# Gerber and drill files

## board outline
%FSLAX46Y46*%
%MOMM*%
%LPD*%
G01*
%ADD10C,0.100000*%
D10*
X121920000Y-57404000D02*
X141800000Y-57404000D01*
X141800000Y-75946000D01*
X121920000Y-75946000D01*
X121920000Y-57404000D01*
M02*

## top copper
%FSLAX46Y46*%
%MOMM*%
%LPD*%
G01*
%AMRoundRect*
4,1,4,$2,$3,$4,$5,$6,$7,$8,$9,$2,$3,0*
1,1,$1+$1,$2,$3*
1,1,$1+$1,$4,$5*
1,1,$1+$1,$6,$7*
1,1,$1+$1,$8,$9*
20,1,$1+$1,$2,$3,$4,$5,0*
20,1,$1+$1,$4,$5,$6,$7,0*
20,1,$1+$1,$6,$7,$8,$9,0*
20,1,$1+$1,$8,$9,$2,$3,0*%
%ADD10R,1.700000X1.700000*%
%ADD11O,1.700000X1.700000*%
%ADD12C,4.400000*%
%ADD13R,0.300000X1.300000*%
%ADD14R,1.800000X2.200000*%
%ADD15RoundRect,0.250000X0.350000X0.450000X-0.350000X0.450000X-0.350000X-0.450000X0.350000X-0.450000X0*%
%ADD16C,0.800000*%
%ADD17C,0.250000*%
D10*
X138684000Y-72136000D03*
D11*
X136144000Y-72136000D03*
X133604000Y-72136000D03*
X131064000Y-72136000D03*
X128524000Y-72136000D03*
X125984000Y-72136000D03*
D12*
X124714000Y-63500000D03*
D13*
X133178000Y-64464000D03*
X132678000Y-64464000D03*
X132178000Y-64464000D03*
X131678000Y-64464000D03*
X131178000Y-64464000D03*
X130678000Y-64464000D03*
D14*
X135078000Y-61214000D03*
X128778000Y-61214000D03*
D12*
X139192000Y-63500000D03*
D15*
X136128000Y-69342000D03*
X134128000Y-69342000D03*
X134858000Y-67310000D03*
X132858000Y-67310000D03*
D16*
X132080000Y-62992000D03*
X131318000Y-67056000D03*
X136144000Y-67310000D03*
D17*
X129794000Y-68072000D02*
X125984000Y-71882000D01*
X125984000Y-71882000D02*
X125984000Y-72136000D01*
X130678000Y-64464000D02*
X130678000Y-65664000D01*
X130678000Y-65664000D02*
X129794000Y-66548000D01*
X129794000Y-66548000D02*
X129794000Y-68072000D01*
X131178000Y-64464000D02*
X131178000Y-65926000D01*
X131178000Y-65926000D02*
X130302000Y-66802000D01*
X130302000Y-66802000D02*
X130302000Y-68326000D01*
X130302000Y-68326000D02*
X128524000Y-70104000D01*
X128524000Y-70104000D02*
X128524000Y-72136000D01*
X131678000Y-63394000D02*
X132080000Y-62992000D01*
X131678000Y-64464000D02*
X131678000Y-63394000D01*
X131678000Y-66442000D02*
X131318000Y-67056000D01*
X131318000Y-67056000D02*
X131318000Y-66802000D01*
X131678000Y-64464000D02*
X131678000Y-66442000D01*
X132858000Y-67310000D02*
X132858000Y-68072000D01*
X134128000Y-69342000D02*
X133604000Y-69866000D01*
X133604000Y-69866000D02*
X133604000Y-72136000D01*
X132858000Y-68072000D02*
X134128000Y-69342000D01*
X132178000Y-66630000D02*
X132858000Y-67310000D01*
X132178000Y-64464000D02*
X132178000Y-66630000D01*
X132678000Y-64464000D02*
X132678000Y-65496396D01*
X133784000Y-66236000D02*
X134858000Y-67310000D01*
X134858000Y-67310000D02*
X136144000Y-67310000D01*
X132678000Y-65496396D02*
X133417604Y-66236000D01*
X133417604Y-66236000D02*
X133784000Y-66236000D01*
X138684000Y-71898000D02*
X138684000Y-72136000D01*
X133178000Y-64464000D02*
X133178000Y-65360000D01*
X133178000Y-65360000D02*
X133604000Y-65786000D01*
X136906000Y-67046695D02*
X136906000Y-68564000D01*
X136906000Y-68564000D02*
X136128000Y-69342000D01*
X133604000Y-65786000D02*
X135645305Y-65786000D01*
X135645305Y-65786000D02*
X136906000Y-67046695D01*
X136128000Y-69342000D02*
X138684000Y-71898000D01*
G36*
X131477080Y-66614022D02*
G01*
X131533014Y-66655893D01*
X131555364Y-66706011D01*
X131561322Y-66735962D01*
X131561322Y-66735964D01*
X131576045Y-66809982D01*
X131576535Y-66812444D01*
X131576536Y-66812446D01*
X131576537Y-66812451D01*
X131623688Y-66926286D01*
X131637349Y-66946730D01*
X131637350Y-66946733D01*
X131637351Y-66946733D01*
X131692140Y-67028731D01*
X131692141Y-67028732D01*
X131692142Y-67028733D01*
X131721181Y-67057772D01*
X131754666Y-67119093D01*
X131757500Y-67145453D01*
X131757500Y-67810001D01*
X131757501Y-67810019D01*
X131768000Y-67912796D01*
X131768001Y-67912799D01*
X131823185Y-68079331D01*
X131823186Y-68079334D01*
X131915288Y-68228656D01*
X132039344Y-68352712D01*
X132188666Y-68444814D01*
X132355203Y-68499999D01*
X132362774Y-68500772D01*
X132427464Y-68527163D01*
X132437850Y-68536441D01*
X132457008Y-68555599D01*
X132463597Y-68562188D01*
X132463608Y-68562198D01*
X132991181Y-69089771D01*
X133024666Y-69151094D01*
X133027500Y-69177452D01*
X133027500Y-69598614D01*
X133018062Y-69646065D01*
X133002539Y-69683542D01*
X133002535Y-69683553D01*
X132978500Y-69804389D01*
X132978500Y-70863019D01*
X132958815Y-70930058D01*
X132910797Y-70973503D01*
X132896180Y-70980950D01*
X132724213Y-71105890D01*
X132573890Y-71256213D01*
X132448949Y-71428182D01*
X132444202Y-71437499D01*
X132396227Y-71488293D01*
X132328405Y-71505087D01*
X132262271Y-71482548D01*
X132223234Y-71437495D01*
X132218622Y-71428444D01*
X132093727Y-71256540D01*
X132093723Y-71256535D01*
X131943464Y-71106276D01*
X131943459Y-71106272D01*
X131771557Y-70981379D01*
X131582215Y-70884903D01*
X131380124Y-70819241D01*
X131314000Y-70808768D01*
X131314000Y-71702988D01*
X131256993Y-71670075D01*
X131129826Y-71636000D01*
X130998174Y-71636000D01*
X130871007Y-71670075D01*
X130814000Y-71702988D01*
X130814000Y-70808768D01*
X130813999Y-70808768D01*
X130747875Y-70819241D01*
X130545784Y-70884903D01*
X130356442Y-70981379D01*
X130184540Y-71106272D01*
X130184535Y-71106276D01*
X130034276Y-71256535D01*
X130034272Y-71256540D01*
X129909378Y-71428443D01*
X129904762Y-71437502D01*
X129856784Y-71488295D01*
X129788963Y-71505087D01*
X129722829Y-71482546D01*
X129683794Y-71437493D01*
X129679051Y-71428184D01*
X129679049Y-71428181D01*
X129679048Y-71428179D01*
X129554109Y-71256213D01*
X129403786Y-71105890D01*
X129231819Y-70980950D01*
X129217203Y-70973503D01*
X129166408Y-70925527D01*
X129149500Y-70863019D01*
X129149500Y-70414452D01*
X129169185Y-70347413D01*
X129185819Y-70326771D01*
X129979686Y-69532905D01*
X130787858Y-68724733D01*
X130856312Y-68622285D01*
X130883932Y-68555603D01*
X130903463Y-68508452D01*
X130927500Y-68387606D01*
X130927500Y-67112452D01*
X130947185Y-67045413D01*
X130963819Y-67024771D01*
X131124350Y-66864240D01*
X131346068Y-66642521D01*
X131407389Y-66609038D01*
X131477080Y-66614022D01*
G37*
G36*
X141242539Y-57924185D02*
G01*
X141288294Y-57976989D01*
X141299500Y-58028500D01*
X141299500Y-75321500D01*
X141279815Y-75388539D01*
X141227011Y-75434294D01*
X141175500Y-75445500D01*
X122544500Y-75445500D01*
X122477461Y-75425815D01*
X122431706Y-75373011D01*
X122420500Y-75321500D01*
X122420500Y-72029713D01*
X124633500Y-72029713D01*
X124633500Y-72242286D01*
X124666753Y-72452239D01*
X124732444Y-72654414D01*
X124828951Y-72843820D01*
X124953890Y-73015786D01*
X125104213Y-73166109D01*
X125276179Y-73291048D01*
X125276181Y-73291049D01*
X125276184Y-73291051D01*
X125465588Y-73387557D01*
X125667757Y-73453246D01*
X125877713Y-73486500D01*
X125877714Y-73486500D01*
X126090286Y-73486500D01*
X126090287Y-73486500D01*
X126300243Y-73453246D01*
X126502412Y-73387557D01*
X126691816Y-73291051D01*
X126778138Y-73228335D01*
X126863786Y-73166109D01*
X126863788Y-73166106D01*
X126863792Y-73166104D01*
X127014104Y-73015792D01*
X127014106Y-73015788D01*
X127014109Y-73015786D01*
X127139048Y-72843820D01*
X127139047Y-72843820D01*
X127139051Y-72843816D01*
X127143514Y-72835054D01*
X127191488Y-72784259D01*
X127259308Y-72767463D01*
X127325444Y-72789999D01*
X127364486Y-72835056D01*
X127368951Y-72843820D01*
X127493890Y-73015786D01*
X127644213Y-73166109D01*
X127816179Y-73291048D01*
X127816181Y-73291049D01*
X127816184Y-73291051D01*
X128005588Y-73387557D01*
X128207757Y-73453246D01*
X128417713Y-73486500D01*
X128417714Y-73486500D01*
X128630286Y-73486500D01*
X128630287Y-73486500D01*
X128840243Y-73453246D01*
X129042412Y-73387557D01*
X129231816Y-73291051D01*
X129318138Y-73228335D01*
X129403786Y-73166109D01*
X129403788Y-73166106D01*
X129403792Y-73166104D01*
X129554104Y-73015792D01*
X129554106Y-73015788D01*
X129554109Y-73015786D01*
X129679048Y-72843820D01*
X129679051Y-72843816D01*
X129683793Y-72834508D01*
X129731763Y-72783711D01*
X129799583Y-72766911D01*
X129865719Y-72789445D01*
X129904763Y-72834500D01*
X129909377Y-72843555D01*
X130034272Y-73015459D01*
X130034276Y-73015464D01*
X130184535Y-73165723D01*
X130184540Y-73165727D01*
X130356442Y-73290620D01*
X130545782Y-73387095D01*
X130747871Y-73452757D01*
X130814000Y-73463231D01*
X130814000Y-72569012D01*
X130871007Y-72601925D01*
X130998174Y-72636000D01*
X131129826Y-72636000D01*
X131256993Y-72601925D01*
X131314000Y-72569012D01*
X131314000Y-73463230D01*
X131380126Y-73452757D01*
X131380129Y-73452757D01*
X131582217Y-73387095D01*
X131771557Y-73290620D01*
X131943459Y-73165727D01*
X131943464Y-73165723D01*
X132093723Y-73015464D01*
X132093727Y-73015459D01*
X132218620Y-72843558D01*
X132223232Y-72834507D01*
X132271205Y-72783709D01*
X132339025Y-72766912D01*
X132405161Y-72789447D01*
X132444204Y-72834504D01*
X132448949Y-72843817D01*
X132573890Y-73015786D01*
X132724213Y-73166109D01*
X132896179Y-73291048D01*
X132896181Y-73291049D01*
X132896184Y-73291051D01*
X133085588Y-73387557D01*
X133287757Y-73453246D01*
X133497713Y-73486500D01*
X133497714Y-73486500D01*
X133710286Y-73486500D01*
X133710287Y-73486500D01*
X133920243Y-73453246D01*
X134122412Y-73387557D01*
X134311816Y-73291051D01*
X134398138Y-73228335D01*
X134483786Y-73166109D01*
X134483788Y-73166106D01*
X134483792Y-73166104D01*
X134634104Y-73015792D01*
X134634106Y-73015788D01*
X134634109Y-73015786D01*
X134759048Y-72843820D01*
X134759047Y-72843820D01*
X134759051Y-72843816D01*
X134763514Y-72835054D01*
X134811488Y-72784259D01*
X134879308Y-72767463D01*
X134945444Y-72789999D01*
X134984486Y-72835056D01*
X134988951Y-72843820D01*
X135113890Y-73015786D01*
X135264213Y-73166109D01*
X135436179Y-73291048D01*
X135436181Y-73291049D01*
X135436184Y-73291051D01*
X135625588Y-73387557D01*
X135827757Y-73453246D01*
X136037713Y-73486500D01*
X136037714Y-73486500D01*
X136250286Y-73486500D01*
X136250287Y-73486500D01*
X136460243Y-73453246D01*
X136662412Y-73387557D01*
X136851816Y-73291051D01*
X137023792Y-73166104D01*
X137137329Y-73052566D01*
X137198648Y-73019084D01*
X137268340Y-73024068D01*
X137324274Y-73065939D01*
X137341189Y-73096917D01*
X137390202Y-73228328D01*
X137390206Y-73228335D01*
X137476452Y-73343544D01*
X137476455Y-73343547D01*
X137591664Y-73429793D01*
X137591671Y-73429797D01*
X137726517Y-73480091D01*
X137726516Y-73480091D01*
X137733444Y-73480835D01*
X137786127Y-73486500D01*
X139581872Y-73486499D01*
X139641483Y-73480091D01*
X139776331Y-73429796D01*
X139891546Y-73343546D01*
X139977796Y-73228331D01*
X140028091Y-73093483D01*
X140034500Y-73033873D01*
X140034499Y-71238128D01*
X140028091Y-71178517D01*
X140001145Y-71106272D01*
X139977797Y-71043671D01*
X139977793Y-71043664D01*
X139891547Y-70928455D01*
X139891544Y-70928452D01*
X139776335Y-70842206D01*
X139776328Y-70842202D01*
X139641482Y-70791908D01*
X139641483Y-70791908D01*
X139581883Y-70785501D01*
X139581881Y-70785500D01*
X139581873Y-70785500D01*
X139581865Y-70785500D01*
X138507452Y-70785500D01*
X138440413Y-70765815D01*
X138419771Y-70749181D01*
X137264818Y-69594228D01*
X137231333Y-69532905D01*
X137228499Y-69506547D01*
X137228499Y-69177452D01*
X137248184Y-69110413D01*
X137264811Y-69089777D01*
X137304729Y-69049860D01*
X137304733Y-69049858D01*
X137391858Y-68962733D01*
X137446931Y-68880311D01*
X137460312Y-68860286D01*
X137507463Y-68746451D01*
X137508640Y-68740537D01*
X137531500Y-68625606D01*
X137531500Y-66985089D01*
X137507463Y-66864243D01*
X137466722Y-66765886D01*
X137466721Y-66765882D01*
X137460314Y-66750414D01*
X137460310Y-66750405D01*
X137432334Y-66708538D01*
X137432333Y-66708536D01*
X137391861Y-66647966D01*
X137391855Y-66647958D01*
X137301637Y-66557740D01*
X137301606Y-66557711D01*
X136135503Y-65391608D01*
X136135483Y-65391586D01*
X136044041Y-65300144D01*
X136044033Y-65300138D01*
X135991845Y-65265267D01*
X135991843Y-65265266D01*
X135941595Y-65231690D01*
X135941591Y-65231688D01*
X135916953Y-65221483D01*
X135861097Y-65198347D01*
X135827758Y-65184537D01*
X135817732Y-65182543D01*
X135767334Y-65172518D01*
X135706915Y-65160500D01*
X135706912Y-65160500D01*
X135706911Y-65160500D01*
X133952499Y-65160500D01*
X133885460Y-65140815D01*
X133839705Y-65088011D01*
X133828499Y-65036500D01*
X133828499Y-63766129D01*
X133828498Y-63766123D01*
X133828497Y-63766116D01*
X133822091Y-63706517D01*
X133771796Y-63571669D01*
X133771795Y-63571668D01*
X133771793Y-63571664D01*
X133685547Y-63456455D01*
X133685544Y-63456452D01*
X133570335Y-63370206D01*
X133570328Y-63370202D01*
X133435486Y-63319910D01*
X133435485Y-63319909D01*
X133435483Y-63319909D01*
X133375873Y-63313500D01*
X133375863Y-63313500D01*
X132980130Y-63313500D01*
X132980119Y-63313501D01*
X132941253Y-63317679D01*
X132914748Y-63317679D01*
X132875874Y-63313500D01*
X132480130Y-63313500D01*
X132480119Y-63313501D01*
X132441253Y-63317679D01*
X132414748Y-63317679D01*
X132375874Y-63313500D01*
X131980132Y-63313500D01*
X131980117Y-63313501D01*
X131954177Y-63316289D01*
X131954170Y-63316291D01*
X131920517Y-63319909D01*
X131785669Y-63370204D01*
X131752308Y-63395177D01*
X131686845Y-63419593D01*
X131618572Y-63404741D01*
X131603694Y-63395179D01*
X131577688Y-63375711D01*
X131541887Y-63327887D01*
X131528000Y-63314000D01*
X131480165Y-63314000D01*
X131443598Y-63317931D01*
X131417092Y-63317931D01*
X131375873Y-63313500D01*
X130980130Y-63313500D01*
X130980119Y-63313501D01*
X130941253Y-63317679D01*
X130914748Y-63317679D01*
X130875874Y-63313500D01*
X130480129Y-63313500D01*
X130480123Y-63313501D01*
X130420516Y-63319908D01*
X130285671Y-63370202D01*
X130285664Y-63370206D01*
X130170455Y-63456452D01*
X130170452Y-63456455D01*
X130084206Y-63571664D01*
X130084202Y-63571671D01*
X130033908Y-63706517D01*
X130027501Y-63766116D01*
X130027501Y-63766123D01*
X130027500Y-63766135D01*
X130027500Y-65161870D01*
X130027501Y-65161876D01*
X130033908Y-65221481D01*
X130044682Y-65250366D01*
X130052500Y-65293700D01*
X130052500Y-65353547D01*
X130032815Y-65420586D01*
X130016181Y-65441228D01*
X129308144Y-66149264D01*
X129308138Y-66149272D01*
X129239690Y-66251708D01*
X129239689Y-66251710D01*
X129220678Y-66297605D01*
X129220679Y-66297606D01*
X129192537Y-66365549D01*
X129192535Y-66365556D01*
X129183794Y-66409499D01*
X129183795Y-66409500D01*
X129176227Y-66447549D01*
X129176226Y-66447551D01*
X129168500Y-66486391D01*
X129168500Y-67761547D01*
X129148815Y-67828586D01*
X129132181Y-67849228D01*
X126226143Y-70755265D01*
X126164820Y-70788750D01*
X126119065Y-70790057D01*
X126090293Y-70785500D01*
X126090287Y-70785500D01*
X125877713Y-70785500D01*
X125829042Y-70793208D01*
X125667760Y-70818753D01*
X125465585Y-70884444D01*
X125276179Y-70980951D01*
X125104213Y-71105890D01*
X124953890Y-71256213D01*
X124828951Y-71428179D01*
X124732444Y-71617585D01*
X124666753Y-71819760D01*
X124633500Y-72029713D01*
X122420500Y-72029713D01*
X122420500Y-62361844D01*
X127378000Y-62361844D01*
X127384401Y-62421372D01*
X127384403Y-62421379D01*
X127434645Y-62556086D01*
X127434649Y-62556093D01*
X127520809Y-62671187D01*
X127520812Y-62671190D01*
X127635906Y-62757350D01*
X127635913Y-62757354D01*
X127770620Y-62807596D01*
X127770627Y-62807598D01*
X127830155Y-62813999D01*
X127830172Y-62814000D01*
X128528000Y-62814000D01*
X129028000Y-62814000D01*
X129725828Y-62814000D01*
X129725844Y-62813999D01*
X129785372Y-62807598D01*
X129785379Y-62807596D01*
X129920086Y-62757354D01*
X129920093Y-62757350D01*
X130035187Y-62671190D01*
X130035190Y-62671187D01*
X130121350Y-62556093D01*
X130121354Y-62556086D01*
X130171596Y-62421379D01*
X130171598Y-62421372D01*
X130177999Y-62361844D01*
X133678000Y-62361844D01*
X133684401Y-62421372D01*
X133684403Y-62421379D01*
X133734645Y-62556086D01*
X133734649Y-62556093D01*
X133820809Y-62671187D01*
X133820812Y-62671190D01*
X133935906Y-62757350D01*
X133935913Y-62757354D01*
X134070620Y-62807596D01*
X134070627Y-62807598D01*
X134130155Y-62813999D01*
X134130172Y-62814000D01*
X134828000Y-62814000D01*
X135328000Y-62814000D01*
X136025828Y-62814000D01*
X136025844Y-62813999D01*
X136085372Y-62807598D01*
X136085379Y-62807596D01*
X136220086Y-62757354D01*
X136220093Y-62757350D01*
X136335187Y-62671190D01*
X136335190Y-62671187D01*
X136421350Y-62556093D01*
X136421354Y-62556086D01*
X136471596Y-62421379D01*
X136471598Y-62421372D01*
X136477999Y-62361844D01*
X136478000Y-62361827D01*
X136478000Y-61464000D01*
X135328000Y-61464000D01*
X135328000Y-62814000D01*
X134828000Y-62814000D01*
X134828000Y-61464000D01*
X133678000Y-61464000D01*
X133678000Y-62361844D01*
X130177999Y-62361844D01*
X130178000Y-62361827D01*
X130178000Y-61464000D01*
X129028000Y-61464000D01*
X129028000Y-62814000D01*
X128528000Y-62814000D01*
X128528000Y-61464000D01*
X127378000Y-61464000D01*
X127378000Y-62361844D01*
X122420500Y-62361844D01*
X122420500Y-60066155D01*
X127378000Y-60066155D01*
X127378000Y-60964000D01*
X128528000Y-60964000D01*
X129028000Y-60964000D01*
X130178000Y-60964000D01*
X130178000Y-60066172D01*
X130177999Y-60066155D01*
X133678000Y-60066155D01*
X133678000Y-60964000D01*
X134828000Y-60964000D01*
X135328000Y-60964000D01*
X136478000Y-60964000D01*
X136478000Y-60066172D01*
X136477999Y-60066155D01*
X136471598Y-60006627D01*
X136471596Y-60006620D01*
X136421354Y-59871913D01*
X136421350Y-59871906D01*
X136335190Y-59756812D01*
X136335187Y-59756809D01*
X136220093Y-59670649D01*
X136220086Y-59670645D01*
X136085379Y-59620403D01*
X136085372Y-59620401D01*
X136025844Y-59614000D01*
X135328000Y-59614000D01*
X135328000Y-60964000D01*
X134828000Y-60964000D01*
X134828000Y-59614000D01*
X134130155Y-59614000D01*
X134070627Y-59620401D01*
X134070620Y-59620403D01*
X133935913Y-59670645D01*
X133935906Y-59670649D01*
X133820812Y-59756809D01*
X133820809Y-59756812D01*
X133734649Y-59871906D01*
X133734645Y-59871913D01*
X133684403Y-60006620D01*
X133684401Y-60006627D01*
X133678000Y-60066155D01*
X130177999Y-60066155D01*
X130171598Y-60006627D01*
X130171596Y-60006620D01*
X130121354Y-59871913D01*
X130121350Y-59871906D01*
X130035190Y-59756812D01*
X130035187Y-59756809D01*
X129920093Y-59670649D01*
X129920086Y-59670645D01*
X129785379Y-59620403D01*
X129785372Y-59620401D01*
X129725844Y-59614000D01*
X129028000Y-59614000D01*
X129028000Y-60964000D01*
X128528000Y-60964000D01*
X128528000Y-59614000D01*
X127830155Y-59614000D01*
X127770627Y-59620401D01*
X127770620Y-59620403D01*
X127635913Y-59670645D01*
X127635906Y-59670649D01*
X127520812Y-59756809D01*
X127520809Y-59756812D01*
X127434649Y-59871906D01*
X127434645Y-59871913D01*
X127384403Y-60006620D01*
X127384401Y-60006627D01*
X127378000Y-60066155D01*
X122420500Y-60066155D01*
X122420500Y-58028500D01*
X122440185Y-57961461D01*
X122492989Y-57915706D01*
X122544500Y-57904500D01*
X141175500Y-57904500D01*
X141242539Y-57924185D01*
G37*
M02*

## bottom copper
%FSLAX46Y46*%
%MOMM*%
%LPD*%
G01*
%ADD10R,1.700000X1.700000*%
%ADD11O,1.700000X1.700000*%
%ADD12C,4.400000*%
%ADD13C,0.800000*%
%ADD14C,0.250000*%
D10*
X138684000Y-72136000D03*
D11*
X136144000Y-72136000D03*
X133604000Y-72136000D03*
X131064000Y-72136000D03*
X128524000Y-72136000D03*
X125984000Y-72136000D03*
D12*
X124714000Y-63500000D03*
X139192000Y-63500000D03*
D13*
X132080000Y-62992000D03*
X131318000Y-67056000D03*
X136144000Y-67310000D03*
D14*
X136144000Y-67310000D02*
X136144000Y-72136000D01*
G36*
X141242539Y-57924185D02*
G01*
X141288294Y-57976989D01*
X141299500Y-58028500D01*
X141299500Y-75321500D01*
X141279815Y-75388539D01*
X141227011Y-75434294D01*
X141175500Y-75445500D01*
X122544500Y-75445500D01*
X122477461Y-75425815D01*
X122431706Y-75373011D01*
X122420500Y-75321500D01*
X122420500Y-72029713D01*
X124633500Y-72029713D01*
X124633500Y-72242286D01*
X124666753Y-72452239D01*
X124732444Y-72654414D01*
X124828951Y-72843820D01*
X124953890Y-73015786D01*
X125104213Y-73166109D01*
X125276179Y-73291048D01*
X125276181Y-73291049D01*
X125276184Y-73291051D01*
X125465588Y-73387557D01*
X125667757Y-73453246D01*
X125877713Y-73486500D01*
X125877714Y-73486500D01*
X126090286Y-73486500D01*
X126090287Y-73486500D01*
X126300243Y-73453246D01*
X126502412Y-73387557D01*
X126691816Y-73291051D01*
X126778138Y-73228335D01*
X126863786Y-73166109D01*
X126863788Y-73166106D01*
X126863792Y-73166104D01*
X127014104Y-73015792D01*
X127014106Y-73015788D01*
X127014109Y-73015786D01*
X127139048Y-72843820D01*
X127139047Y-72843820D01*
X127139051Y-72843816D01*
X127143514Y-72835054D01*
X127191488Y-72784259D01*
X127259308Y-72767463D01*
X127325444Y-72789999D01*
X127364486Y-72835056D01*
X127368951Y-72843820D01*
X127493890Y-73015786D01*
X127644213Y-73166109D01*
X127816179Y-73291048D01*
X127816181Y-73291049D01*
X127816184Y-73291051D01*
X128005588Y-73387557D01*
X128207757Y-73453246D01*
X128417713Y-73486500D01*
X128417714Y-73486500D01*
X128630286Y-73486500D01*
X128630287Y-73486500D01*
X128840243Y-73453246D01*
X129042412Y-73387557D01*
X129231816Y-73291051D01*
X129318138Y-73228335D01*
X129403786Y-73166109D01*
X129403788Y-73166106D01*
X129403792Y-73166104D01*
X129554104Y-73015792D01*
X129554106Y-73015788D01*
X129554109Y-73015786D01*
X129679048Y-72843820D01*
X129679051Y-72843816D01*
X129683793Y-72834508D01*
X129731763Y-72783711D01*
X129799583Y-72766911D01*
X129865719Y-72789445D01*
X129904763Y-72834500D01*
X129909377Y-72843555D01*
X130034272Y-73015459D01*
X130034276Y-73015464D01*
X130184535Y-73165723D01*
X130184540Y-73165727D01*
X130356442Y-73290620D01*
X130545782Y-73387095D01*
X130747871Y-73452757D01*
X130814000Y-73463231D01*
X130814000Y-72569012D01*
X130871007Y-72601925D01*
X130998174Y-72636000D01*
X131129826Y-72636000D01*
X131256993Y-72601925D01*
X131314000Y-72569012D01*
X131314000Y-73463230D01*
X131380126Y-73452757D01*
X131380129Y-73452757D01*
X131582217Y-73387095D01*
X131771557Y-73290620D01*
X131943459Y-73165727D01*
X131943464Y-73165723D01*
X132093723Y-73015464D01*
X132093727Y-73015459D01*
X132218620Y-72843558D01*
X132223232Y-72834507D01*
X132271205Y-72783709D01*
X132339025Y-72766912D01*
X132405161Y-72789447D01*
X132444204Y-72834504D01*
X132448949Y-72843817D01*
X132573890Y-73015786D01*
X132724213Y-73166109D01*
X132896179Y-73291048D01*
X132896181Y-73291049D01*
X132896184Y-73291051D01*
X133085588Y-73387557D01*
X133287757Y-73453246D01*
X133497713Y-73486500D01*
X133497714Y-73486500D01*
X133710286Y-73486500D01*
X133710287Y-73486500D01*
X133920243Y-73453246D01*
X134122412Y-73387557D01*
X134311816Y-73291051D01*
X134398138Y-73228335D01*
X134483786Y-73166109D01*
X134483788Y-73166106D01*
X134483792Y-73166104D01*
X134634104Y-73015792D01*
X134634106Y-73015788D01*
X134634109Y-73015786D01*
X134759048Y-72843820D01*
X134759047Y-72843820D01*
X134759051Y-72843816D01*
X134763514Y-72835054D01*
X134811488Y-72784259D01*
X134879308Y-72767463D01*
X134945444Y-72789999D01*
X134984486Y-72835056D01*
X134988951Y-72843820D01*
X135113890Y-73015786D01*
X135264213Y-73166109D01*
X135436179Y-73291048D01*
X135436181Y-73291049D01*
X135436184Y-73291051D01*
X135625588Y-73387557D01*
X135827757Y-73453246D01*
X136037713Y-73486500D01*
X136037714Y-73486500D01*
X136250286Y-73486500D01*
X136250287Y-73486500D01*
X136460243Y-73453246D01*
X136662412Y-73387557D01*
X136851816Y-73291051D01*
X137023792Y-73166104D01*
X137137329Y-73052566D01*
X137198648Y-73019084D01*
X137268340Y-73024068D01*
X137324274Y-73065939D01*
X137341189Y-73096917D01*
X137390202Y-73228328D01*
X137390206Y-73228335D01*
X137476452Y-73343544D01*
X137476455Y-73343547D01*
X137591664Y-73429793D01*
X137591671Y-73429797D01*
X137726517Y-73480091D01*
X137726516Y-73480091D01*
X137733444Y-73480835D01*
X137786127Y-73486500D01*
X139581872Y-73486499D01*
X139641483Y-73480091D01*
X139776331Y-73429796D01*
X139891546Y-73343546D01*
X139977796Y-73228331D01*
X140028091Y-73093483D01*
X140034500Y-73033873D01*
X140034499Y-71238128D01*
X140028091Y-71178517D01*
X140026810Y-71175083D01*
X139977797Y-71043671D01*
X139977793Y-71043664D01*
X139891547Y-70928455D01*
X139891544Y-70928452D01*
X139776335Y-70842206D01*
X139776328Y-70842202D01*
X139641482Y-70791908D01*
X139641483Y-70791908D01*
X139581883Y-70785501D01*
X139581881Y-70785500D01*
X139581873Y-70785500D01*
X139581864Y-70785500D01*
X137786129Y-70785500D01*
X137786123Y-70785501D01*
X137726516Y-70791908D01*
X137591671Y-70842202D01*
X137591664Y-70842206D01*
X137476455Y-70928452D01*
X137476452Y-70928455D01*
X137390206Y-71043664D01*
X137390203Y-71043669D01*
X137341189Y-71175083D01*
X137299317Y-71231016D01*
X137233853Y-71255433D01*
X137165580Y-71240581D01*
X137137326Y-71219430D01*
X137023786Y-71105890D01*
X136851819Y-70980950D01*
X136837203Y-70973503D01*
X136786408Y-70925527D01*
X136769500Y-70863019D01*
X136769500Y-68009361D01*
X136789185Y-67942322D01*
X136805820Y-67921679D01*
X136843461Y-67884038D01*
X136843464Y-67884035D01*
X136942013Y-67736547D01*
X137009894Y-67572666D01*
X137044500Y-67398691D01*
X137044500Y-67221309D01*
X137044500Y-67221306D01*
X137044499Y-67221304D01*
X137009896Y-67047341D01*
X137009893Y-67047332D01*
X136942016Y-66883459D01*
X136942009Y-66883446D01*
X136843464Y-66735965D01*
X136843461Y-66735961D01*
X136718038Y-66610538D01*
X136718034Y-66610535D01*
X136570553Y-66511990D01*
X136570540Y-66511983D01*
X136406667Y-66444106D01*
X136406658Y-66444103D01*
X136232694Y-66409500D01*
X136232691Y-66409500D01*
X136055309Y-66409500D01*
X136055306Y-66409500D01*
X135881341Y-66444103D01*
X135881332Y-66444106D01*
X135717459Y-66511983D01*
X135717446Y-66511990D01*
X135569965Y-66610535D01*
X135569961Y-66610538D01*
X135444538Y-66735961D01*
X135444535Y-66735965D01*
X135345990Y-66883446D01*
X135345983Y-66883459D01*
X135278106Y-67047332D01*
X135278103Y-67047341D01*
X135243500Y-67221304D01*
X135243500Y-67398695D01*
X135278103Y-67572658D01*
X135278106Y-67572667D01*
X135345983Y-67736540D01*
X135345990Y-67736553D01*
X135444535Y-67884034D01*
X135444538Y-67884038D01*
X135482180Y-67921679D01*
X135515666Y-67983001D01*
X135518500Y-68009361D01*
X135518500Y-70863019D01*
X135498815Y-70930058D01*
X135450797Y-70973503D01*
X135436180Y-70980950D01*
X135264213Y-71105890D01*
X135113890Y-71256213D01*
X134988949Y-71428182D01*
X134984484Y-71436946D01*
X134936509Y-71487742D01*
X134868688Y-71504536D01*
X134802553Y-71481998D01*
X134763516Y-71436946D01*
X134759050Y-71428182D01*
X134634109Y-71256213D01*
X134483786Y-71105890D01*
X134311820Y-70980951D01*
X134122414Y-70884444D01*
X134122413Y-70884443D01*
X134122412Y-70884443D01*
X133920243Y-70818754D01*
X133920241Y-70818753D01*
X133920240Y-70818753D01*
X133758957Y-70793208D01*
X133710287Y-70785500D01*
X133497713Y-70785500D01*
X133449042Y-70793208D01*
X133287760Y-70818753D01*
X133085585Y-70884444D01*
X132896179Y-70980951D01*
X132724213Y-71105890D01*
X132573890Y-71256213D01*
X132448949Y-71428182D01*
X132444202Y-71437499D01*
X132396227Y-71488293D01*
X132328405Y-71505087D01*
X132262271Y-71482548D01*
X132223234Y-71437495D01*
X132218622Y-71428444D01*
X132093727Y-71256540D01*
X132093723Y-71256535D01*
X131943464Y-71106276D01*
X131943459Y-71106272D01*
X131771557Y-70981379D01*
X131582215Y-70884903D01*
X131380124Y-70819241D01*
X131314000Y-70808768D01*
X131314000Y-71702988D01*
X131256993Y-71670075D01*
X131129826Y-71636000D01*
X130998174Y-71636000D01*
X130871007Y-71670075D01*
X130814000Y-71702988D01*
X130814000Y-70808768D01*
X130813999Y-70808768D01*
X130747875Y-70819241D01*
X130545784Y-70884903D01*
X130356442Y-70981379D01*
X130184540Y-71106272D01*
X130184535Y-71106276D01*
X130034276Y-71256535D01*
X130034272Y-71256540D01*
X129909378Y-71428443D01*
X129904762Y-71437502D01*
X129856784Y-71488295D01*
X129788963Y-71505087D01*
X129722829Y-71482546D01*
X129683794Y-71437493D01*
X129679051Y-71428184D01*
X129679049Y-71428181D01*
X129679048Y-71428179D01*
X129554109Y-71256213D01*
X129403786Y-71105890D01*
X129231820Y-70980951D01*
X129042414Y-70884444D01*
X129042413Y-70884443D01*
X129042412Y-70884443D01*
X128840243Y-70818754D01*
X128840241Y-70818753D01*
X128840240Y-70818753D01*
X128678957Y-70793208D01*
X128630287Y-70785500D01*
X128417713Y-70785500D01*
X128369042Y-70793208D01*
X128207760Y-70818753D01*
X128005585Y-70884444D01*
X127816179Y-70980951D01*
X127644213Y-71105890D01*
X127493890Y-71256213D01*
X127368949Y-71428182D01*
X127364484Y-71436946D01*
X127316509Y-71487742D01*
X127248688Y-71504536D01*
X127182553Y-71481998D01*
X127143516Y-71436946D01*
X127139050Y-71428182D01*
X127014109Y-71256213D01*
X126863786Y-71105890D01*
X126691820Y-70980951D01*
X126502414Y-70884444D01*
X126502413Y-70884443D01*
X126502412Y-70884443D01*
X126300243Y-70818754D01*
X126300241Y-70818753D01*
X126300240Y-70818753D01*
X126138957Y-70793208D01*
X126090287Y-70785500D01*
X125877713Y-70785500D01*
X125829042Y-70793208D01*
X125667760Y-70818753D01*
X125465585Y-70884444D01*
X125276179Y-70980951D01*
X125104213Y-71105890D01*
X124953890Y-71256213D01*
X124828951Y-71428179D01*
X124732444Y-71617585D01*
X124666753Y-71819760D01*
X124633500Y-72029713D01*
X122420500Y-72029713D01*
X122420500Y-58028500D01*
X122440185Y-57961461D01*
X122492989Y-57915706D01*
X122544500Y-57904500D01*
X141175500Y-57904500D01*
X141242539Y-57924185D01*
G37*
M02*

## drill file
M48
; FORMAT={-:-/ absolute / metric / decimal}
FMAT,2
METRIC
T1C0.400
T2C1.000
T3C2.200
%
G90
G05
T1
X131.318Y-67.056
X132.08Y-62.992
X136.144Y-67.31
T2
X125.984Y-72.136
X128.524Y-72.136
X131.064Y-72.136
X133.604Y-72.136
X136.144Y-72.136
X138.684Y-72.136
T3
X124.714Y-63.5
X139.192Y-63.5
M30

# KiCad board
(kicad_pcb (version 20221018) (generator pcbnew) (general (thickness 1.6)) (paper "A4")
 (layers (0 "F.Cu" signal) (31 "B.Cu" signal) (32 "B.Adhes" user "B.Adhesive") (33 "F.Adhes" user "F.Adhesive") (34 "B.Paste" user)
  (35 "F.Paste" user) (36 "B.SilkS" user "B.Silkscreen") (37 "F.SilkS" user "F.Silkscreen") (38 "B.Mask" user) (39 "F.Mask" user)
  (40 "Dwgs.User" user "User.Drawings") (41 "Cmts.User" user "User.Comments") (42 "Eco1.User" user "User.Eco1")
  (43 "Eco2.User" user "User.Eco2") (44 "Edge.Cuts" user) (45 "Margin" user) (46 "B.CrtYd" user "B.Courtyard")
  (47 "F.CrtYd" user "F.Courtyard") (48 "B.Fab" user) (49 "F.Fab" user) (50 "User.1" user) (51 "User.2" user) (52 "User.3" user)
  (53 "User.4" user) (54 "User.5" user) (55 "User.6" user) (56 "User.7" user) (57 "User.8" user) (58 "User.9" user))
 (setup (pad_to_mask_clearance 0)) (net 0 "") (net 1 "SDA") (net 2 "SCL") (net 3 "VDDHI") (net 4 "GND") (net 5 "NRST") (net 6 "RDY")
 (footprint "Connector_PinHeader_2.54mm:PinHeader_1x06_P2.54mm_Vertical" (layer "F.Cu") (at 138.684 72.136 -90)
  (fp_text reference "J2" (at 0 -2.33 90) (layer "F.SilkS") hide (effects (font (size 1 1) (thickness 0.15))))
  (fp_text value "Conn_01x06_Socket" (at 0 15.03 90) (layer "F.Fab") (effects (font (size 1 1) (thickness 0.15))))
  (pad "1" thru_hole rect (at 0 0 270) (size 1.7 1.7) (drill 1) (layers "*.Cu" "*.Mask") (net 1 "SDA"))
  (pad "2" thru_hole oval (at 0 2.54 270) (size 1.7 1.7) (drill 1) (layers "*.Cu" "*.Mask") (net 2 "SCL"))
  (pad "3" thru_hole oval (at 0 5.08 270) (size 1.7 1.7) (drill 1) (layers "*.Cu" "*.Mask") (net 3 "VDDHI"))
  (pad "4" thru_hole oval (at 0 7.62 270) (size 1.7 1.7) (drill 1) (layers "*.Cu" "*.Mask") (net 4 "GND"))
  (pad "5" thru_hole oval (at 0 10.16 270) (size 1.7 1.7) (drill 1) (layers "*.Cu" "*.Mask") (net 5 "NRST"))
  (pad "6" thru_hole oval (at 0 12.7 270) (size 1.7 1.7) (drill 1) (layers "*.Cu" "*.Mask") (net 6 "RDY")))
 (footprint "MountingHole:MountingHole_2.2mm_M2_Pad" (layer "F.Cu") (at 124.714 63.5)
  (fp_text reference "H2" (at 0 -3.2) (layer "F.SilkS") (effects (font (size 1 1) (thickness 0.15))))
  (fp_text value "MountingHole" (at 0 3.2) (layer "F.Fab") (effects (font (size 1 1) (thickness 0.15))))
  (pad "1" thru_hole circle (at 0 0) (size 4.4 4.4) (drill 2.2) (layers "*.Cu" "*.Mask") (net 4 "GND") (zone_connect 2)))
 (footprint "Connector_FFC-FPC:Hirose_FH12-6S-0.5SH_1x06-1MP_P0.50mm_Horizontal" (layer "F.Cu") (at 131.928 62.614 180)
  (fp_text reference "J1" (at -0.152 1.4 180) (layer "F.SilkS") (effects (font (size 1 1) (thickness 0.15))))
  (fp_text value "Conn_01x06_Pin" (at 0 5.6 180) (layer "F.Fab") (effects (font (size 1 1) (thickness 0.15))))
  (pad "1" smd rect (at -1.25 -1.85 180) (size 0.3 1.3) (layers "F.Cu" "F.Paste" "F.Mask") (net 1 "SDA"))
  (pad "2" smd rect (at -0.75 -1.85 180) (size 0.3 1.3) (layers "F.Cu" "F.Paste" "F.Mask") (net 2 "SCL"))
  (pad "3" smd rect (at -0.25 -1.85 180) (size 0.3 1.3) (layers "F.Cu" "F.Paste" "F.Mask") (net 3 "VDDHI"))
  (pad "4" smd rect (at 0.25 -1.85 180) (size 0.3 1.3) (layers "F.Cu" "F.Paste" "F.Mask") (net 4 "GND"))
  (pad "5" smd rect (at 0.75 -1.85 180) (size 0.3 1.3) (layers "F.Cu" "F.Paste" "F.Mask") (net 5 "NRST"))
  (pad "6" smd rect (at 1.25 -1.85 180) (size 0.3 1.3) (layers "F.Cu" "F.Paste" "F.Mask") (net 6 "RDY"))
  (pad "MP" smd rect (at -3.15 1.4 180) (size 1.8 2.2) (layers "F.Cu" "F.Paste" "F.Mask") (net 4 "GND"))
  (pad "MP" smd rect (at 3.15 1.4 180) (size 1.8 2.2) (layers "F.Cu" "F.Paste" "F.Mask") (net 4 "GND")))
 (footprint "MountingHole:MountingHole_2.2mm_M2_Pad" (layer "F.Cu") (at 139.192 63.5)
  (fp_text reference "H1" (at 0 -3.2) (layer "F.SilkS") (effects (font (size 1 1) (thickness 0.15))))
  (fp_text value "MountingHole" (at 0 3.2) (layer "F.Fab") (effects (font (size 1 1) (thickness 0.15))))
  (pad "1" thru_hole circle (at 0 0) (size 4.4 4.4) (drill 2.2) (layers "*.Cu" "*.Mask") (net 4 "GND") (zone_connect 2)))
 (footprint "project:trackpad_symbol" (layer "F.Cu") (at 125.73 68.072)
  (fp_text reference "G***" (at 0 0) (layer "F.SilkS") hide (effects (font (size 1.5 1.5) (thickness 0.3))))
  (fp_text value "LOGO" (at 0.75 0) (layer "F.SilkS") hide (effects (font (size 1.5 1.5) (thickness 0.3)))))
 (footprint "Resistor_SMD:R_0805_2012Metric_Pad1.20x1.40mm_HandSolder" (layer "F.Cu") (at 135.128 69.342 180)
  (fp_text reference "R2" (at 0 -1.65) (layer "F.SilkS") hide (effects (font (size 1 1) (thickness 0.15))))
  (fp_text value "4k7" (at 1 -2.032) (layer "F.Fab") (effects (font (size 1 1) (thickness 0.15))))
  (pad "1" smd roundrect (at -1 0 180) (size 1.2 1.4) (layers "F.Cu" "F.Paste" "F.Mask") (roundrect_rratio 0.2083333333) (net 1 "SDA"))
  (pad "2" smd roundrect (at 1 0 180) (size 1.2 1.4) (layers "F.Cu" "F.Paste" "F.Mask") (roundrect_rratio 0.2083333333) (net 3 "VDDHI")))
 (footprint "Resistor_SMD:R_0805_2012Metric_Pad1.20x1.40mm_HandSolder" (layer "F.Cu") (at 133.858 67.31 180)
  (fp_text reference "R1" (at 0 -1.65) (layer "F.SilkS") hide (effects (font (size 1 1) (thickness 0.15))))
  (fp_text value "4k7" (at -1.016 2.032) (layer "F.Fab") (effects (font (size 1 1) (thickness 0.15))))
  (pad "1" smd roundrect (at -1 0 180) (size 1.2 1.4) (layers "F.Cu" "F.Paste" "F.Mask") (roundrect_rratio 0.2083333333) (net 2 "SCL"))
  (pad "2" smd roundrect (at 1 0 180) (size 1.2 1.4) (layers "F.Cu" "F.Paste" "F.Mask") (roundrect_rratio 0.2083333333) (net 3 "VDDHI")))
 (gr_rect (start 121.92 57.404) (end 141.8 75.946) (stroke (width 0.1) (type default)) (fill none) (layer "Edge.Cuts"))
 (segment (start 129.794 68.072) (end 125.984 71.882) (width 0.25) (layer "F.Cu") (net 6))
 (segment (start 125.984 71.882) (end 125.984 72.136) (width 0.25) (layer "F.Cu") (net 6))
 (segment (start 130.678 64.464) (end 130.678 65.664) (width 0.25) (layer "F.Cu") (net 6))
 (segment (start 130.678 65.664) (end 129.794 66.548) (width 0.25) (layer "F.Cu") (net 6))
 (segment (start 129.794 66.548) (end 129.794 68.072) (width 0.25) (layer "F.Cu") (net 6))
 (segment (start 131.178 64.464) (end 131.178 65.926) (width 0.25) (layer "F.Cu") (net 5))
 (segment (start 131.178 65.926) (end 130.302 66.802) (width 0.25) (layer "F.Cu") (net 5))
 (segment (start 130.302 66.802) (end 130.302 68.326) (width 0.25) (layer "F.Cu") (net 5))
 (segment (start 130.302 68.326) (end 128.524 70.104) (width 0.25) (layer "F.Cu") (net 5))
 (segment (start 128.524 70.104) (end 128.524 72.136) (width 0.25) (layer "F.Cu") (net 5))
 (segment (start 131.678 63.394) (end 132.08 62.992) (width 0.25) (layer "F.Cu") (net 4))
 (segment (start 131.678 64.464) (end 131.678 63.394) (width 0.25) (layer "F.Cu") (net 4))
 (segment (start 131.678 66.442) (end 131.318 67.056) (width 0.25) (layer "F.Cu") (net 4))
 (segment (start 131.318 67.056) (end 131.318 66.802) (width 0.25) (layer "F.Cu") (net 4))
 (segment (start 131.678 64.464) (end 131.678 66.442) (width 0.25) (layer "F.Cu") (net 4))
 (via (at 132.08 62.992) (size 0.8) (drill 0.4) (layers "F.Cu" "B.Cu") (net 4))
 (via (at 131.318 67.056) (size 0.8) (drill 0.4) (layers "F.Cu" "B.Cu") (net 4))
 (segment (start 132.858 67.31) (end 132.858 68.072) (width 0.25) (layer "F.Cu") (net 3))
 (segment (start 134.128 69.342) (end 133.604 69.866) (width 0.25) (layer "F.Cu") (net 3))
 (segment (start 133.604 69.866) (end 133.604 72.136) (width 0.25) (layer "F.Cu") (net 3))
 (segment (start 132.858 68.072) (end 134.128 69.342) (width 0.25) (layer "F.Cu") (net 3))
 (segment (start 132.178 66.63) (end 132.858 67.31) (width 0.25) (layer "F.Cu") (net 3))
 (segment (start 132.178 64.464) (end 132.178 66.63) (width 0.25) (layer "F.Cu") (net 3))
 (segment (start 132.678 64.464) (end 132.678 65.496396) (width 0.25) (layer "F.Cu") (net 2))
 (segment (start 133.784 66.236) (end 134.858 67.31) (width 0.25) (layer "F.Cu") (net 2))
 (segment (start 134.858 67.31) (end 136.144 67.31) (width 0.25) (layer "F.Cu") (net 2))
 (segment (start 132.678 65.496396) (end 133.417604 66.236) (width 0.25) (layer "F.Cu") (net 2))
 (segment (start 133.417604 66.236) (end 133.784 66.236) (width 0.25) (layer "F.Cu") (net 2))
 (via (at 136.144 67.31) (size 0.8) (drill 0.4) (layers "F.Cu" "B.Cu") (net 2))
 (segment (start 136.144 67.31) (end 136.144 72.136) (width 0.25) (layer "B.Cu") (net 2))
 (segment (start 138.684 71.898) (end 138.684 72.136) (width 0.25) (layer "F.Cu") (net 1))
 (segment (start 133.178 64.464) (end 133.178 65.36) (width 0.25) (layer "F.Cu") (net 1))
 (segment (start 133.178 65.36) (end 133.604 65.786) (width 0.25) (layer "F.Cu") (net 1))
 (segment (start 136.906 67.046695) (end 136.906 68.564) (width 0.25) (layer "F.Cu") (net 1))
 (segment (start 136.906 68.564) (end 136.128 69.342) (width 0.25) (layer "F.Cu") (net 1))
 (segment (start 133.604 65.786) (end 135.645305 65.786) (width 0.25) (layer "F.Cu") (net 1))
 (segment (start 135.645305 65.786) (end 136.906 67.046695) (width 0.25) (layer "F.Cu") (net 1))
 (segment (start 136.128 69.342) (end 138.684 71.898) (width 0.25) (layer "F.Cu") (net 1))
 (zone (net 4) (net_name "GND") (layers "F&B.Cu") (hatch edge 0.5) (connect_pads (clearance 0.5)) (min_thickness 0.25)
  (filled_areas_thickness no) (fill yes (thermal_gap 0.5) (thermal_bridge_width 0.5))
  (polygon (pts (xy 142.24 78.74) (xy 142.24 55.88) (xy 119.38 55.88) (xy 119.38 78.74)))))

